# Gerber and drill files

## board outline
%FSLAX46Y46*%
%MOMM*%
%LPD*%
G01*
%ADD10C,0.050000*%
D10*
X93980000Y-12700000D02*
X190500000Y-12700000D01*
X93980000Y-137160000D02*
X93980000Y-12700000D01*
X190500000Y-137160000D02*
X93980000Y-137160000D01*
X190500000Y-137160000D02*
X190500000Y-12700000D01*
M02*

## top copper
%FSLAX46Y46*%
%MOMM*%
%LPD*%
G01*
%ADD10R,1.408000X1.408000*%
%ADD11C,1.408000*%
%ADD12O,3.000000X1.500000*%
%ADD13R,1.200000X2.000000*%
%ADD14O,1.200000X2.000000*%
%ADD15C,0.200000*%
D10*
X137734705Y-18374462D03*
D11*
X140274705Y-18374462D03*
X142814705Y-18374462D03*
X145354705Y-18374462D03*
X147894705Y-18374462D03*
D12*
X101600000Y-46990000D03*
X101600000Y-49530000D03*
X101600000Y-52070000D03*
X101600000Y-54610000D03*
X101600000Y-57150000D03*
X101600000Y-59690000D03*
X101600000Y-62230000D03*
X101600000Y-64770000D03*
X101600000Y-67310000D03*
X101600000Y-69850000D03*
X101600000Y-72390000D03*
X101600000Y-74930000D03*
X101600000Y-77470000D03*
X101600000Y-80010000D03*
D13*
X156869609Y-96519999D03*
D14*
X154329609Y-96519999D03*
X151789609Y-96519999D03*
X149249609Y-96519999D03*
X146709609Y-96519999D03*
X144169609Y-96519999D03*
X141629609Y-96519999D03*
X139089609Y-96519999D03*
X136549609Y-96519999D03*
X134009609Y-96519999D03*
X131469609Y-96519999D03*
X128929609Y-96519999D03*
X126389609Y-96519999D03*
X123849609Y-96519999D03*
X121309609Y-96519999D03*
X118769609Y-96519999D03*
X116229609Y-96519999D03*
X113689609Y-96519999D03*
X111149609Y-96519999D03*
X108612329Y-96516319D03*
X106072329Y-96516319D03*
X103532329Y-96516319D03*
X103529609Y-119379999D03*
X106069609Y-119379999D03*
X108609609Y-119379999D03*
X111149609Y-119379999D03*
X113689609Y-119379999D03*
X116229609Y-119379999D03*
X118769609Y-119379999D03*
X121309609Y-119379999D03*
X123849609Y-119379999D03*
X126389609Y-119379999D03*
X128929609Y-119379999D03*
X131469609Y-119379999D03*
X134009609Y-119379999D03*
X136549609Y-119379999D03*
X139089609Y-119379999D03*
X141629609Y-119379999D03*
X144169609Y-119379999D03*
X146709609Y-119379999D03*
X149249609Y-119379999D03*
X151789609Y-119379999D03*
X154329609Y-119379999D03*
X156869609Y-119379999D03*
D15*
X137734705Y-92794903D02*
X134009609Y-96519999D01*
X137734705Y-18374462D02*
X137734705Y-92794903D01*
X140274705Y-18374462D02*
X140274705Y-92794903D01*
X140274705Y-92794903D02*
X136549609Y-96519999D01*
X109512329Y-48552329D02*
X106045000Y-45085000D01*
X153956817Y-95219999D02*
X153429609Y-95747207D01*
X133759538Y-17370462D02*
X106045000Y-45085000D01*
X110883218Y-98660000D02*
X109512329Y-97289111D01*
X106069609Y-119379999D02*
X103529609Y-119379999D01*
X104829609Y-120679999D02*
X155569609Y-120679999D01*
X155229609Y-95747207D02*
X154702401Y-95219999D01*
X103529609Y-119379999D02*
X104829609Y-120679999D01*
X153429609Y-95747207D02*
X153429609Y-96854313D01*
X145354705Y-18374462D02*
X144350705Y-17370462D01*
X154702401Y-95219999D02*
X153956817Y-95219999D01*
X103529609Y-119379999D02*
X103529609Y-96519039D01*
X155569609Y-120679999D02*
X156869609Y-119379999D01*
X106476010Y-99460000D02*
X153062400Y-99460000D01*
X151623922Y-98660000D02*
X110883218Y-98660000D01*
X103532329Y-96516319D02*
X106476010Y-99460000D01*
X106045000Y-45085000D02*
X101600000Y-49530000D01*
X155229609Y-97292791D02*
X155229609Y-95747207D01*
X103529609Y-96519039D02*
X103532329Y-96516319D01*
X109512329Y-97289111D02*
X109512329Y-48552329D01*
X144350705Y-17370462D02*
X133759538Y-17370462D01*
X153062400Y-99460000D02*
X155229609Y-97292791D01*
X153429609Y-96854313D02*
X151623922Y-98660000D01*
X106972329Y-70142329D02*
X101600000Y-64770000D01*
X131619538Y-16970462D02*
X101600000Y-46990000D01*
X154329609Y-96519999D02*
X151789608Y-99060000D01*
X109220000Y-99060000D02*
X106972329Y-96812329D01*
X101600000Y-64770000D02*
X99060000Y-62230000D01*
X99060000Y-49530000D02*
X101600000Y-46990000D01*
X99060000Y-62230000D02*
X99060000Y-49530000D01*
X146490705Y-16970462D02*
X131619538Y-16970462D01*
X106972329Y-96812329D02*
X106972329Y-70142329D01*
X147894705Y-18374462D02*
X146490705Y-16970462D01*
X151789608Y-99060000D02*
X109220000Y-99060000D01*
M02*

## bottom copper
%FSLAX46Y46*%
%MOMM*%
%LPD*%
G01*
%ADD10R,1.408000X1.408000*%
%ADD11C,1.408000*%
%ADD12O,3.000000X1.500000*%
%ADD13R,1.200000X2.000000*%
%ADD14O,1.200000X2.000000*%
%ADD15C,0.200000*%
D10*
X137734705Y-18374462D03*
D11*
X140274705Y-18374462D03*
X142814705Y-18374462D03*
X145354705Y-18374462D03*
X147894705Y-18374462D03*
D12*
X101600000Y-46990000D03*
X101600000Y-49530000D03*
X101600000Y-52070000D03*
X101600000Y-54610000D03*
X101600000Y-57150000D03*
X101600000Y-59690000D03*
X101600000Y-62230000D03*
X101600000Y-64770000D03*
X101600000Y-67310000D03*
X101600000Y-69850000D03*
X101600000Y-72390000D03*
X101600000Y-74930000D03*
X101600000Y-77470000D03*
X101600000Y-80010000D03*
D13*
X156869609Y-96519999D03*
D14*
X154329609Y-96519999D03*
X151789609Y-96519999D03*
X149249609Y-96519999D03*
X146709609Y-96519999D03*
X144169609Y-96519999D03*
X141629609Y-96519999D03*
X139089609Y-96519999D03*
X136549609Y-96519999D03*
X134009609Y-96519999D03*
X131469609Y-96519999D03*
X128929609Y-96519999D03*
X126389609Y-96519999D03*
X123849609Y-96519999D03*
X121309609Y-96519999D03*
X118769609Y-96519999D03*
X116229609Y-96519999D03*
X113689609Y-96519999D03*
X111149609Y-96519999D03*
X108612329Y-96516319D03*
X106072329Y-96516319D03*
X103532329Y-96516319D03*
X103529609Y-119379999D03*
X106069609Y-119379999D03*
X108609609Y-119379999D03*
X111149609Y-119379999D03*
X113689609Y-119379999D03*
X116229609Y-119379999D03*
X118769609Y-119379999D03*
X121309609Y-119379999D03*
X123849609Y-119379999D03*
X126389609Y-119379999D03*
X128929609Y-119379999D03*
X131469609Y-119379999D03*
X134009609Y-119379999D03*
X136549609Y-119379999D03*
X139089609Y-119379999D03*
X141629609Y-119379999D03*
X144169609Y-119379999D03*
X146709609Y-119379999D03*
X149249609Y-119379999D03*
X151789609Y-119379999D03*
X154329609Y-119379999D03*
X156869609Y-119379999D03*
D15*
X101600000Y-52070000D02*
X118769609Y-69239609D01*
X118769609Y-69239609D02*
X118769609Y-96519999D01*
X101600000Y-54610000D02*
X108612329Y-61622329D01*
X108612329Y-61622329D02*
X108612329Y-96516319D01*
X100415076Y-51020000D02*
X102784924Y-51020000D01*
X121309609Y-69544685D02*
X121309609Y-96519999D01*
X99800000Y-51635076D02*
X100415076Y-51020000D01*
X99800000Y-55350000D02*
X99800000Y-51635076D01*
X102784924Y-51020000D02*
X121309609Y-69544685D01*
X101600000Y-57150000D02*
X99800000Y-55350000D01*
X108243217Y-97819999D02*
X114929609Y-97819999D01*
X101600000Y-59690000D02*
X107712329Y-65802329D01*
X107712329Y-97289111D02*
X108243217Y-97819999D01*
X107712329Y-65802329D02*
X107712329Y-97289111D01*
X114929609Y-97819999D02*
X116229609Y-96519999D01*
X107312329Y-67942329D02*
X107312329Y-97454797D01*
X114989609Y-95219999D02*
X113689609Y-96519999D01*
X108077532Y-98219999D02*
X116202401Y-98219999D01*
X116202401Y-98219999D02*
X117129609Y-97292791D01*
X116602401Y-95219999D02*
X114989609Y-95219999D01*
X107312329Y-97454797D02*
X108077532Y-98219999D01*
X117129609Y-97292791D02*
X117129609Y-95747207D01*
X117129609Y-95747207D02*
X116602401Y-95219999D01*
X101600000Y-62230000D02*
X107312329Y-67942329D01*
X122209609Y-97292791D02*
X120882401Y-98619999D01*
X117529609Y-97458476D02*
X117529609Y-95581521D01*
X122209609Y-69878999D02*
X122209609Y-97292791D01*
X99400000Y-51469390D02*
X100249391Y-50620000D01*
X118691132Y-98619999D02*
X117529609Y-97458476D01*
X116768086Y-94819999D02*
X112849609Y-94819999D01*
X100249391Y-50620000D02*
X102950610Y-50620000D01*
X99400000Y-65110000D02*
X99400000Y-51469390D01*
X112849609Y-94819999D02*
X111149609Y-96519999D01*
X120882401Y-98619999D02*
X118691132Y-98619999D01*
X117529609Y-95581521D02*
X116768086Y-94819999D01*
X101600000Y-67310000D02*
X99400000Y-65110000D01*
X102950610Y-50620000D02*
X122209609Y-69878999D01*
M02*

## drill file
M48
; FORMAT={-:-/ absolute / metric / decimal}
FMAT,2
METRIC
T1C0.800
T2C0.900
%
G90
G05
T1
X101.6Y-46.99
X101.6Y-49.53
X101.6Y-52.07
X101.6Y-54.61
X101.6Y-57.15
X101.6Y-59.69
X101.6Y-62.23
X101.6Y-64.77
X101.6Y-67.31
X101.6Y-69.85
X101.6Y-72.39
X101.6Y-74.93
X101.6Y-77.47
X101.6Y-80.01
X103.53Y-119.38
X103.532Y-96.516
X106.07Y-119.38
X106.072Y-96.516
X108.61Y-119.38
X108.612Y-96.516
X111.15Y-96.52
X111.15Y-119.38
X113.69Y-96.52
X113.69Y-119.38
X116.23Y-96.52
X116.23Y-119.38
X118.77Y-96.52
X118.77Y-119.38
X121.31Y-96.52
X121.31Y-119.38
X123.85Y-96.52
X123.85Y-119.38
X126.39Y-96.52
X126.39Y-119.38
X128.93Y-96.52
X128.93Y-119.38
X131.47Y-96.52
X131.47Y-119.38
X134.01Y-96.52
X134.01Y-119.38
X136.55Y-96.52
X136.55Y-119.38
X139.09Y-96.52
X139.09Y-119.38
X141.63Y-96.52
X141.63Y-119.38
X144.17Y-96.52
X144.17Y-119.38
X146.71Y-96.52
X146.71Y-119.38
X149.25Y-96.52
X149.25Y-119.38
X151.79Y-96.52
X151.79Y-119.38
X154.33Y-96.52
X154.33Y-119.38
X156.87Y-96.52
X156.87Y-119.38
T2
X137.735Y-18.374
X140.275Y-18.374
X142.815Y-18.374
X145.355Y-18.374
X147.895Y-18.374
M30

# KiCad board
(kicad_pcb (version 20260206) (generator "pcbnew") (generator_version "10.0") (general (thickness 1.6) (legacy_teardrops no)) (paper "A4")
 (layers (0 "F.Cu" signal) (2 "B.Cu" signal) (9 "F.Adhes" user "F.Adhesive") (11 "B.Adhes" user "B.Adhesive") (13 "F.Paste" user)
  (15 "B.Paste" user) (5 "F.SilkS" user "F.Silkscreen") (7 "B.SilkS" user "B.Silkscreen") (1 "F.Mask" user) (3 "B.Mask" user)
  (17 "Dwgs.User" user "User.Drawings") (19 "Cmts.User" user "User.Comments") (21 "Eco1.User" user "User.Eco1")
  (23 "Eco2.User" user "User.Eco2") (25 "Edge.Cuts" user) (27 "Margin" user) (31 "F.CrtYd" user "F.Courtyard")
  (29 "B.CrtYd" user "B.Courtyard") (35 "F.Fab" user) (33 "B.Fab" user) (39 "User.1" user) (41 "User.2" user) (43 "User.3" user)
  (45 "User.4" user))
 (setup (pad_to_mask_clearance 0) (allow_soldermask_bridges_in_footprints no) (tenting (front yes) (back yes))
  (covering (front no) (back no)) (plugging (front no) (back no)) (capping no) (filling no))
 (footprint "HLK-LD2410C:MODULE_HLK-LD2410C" (layer "F.Cu") (at 142.764705 24.914462)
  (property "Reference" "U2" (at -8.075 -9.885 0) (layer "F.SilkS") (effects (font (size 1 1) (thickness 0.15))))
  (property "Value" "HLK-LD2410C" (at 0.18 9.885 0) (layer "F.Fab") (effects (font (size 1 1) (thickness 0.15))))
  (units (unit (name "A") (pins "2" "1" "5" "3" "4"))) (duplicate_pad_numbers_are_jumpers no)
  (pad "1" thru_hole rect (at -5.03 -6.54) (size 1.408 1.408) (drill 0.9) (layers "*.Cu" "*.Mask") (remove_unused_layers no) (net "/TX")
   (solder_mask_margin 0.102))
  (pad "2" thru_hole circle (at -2.49 -6.54) (size 1.408 1.408) (drill 0.9) (layers "*.Cu" "*.Mask") (remove_unused_layers no) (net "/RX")
   (solder_mask_margin 0.102))
  (pad "3" thru_hole circle (at 0.05 -6.54) (size 1.408 1.408) (drill 0.9) (layers "*.Cu" "*.Mask") (remove_unused_layers no)
   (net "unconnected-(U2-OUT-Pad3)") (solder_mask_margin 0.102))
  (pad "4" thru_hole circle (at 2.59 -6.54) (size 1.408 1.408) (drill 0.9) (layers "*.Cu" "*.Mask") (remove_unused_layers no) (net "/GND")
   (solder_mask_margin 0.102))
  (pad "5" thru_hole circle (at 5.13 -6.54) (size 1.408 1.408) (drill 0.9) (layers "*.Cu" "*.Mask") (remove_unused_layers no) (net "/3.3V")
   (solder_mask_margin 0.102)))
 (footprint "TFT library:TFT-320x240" (layer "F.Cu") (at 101.6 63.5 -90)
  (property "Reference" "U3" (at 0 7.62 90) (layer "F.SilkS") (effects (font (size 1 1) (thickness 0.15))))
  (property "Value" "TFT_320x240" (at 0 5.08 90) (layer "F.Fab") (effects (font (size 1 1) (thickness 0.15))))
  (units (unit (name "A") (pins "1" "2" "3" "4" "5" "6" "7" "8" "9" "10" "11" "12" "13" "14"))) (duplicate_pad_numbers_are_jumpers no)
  (pad "1" thru_hole oval (at -16.51 0 270) (size 1.5 3) (drill 0.8) (layers "*.Cu" "*.Mask") (remove_unused_layers no) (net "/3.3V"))
  (pad "2" thru_hole oval (at -13.97 0 270) (size 1.5 3) (drill 0.8) (layers "*.Cu" "*.Mask") (remove_unused_layers no) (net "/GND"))
  (pad "3" thru_hole oval (at -11.43 0 270) (size 1.5 3) (drill 0.8) (layers "*.Cu" "*.Mask") (remove_unused_layers no) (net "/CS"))
  (pad "4" thru_hole oval (at -8.89 0 270) (size 1.5 3) (drill 0.8) (layers "*.Cu" "*.Mask") (remove_unused_layers no) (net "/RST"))
  (pad "5" thru_hole oval (at -6.35 0 270) (size 1.5 3) (drill 0.8) (layers "*.Cu" "*.Mask") (remove_unused_layers no) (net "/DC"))
  (pad "6" thru_hole oval (at -3.81 0 270) (size 1.5 3) (drill 0.8) (layers "*.Cu" "*.Mask") (remove_unused_layers no) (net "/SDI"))
  (pad "7" thru_hole oval (at -1.27 0 270) (size 1.5 3) (drill 0.8) (layers "*.Cu" "*.Mask") (remove_unused_layers no) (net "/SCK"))
  (pad "8" thru_hole oval (at 1.27 0 270) (size 1.5 3) (drill 0.8) (layers "*.Cu" "*.Mask") (remove_unused_layers no) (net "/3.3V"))
  (pad "9" thru_hole oval (at 3.81 0 270) (size 1.5 3) (drill 0.8) (layers "*.Cu" "*.Mask") (remove_unused_layers no) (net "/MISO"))
  (pad "10" thru_hole oval (at 6.35 0 270) (size 1.5 3) (drill 0.8) (layers "*.Cu" "*.Mask") (remove_unused_layers no)
   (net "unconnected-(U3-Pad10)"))
  (pad "11" thru_hole oval (at 8.89 0 270) (size 1.5 3) (drill 0.8) (layers "*.Cu" "*.Mask") (remove_unused_layers no)
   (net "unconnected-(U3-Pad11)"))
  (pad "12" thru_hole oval (at 11.43 0 270) (size 1.5 3) (drill 0.8) (layers "*.Cu" "*.Mask") (remove_unused_layers no)
   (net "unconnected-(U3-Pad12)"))
  (pad "13" thru_hole oval (at 13.97 0 270) (size 1.5 3) (drill 0.8) (layers "*.Cu" "*.Mask") (remove_unused_layers no)
   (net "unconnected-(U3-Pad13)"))
  (pad "14" thru_hole oval (at 16.51 0 270) (size 1.5 3) (drill 0.8) (layers "*.Cu" "*.Mask") (remove_unused_layers no)
   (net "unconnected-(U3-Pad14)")))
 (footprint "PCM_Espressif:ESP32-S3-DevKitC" (layer "F.Cu") (at 156.869609 96.519999 -90)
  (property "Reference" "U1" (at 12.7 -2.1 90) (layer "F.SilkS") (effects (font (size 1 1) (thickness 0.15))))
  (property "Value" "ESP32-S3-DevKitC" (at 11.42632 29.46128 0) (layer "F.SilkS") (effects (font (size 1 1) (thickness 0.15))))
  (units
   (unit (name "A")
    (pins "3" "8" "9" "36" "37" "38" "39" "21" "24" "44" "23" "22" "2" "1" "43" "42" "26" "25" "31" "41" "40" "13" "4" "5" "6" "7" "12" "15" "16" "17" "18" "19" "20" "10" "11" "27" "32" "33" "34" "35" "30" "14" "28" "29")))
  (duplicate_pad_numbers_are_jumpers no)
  (pad "1" thru_hole rect (at 0 0 180) (size 1.2 2) (drill 0.8) (layers "*.Cu" "*.Mask") (remove_unused_layers no) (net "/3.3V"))
  (pad "2" thru_hole oval (at 0 2.54 180) (size 1.2 2) (drill 0.8) (layers "*.Cu" "*.Mask") (remove_unused_layers no) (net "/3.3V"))
  (pad "3" thru_hole oval (at 0 5.08 180) (size 1.2 2) (drill 0.8) (layers "*.Cu" "*.Mask") (remove_unused_layers no)
   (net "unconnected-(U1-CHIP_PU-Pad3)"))
  (pad "4" thru_hole oval (at 0 7.62 180) (size 1.2 2) (drill 0.8) (layers "*.Cu" "*.Mask") (remove_unused_layers no)
   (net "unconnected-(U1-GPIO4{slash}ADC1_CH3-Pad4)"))
  (pad "5" thru_hole oval (at 0 10.16 180) (size 1.2 2) (drill 0.8) (layers "*.Cu" "*.Mask") (remove_unused_layers no)
   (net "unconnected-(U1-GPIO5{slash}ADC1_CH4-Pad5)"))
  (pad "6" thru_hole oval (at 0 12.7 180) (size 1.2 2) (drill 0.8) (layers "*.Cu" "*.Mask") (remove_unused_layers no)
   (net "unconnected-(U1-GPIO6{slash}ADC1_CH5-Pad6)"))
  (pad "7" thru_hole oval (at 0 15.24 180) (size 1.2 2) (drill 0.8) (layers "*.Cu" "*.Mask") (remove_unused_layers no)
   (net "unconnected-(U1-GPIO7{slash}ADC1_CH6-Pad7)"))
  (pad "8" thru_hole oval (at 0 17.78 180) (size 1.2 2) (drill 0.8) (layers "*.Cu" "*.Mask") (remove_unused_layers no)
   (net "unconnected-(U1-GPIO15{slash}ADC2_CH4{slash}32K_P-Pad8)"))
  (pad "9" thru_hole oval (at 0 20.32 180) (size 1.2 2) (drill 0.8) (layers "*.Cu" "*.Mask") (remove_unused_layers no) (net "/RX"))
  (pad "10" thru_hole oval (at 0 22.86 180) (size 1.2 2) (drill 0.8) (layers "*.Cu" "*.Mask") (remove_unused_layers no) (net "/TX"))
  (pad "11" thru_hole oval (at 0 25.4 180) (size 1.2 2) (drill 0.8) (layers "*.Cu" "*.Mask") (remove_unused_layers no)
   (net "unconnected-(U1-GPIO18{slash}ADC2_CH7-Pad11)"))
  (pad "12" thru_hole oval (at 0 27.94 180) (size 1.2 2) (drill 0.8) (layers "*.Cu" "*.Mask") (remove_unused_layers no)
   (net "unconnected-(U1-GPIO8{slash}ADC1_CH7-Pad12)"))
  (pad "13" thru_hole oval (at 0 30.48 180) (size 1.2 2) (drill 0.8) (layers "*.Cu" "*.Mask") (remove_unused_layers no)
   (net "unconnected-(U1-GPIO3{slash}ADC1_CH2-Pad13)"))
  (pad "14" thru_hole oval (at 0 33.02 180) (size 1.2 2) (drill 0.8) (layers "*.Cu" "*.Mask") (remove_unused_layers no)
   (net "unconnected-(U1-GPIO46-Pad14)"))
  (pad "15" thru_hole oval (at 0 35.56 180) (size 1.2 2) (drill 0.8) (layers "*.Cu" "*.Mask") (remove_unused_layers no) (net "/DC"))
  (pad "16" thru_hole oval (at 0 38.1 180) (size 1.2 2) (drill 0.8) (layers "*.Cu" "*.Mask") (remove_unused_layers no) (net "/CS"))
  (pad "17" thru_hole oval (at 0 40.64 180) (size 1.2 2) (drill 0.8) (layers "*.Cu" "*.Mask") (remove_unused_layers no) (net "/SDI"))
  (pad "18" thru_hole oval (at 0 43.18 180) (size 1.2 2) (drill 0.8) (layers "*.Cu" "*.Mask") (remove_unused_layers no) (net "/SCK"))
  (pad "19" thru_hole oval (at 0 45.72 180) (size 1.2 2) (drill 0.8) (layers "*.Cu" "*.Mask") (remove_unused_layers no) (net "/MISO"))
  (pad "20" thru_hole oval (at -0.00368 48.25728 180) (size 1.2 2) (drill 0.8) (layers "*.Cu" "*.Mask") (remove_unused_layers no)
   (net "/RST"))
  (pad "21" thru_hole oval (at -0.00368 50.79728 180) (size 1.2 2) (drill 0.8) (layers "*.Cu" "*.Mask") (remove_unused_layers no)
   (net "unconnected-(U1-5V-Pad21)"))
  (pad "22" thru_hole oval (at -0.00368 53.33728 180) (size 1.2 2) (drill 0.8) (layers "*.Cu" "*.Mask") (remove_unused_layers no)
   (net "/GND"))
  (pad "23" thru_hole oval (at 22.86 53.34 180) (size 1.2 2) (drill 0.8) (layers "*.Cu" "*.Mask") (remove_unused_layers no) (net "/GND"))
  (pad "24" thru_hole oval (at 22.86 50.8 180) (size 1.2 2) (drill 0.8) (layers "*.Cu" "*.Mask") (remove_unused_layers no) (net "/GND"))
  (pad "25" thru_hole oval (at 22.86 48.26 180) (size 1.2 2) (drill 0.8) (layers "*.Cu" "*.Mask") (remove_unused_layers no)
   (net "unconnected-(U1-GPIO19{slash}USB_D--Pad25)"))
  (pad "26" thru_hole oval (at 22.86 45.72 180) (size 1.2 2) (drill 0.8) (layers "*.Cu" "*.Mask") (remove_unused_layers no)
   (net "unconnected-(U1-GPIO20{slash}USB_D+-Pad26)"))
  (pad "27" thru_hole oval (at 22.86 43.18 180) (size 1.2 2) (drill 0.8) (layers "*.Cu" "*.Mask") (remove_unused_layers no)
   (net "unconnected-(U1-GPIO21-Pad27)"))
  (pad "28" thru_hole oval (at 22.86 40.64 180) (size 1.2 2) (drill 0.8) (layers "*.Cu" "*.Mask") (remove_unused_layers no)
   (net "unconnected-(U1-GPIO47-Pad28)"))
  (pad "29" thru_hole oval (at 22.86 38.1 180) (size 1.2 2) (drill 0.8) (layers "*.Cu" "*.Mask") (remove_unused_layers no)
   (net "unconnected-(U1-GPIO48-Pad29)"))
  (pad "30" thru_hole oval (at 22.86 35.56 180) (size 1.2 2) (drill 0.8) (layers "*.Cu" "*.Mask") (remove_unused_layers no)
   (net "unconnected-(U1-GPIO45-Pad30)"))
  (pad "31" thru_hole oval (at 22.86 33.02 180) (size 1.2 2) (drill 0.8) (layers "*.Cu" "*.Mask") (remove_unused_layers no)
   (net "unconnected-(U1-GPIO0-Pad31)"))
  (pad "32" thru_hole oval (at 22.86 30.48 180) (size 1.2 2) (drill 0.8) (layers "*.Cu" "*.Mask") (remove_unused_layers no)
   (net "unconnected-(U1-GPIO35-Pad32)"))
  (pad "33" thru_hole oval (at 22.86 27.94 180) (size 1.2 2) (drill 0.8) (layers "*.Cu" "*.Mask") (remove_unused_layers no)
   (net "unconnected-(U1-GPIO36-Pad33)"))
  (pad "34" thru_hole oval (at 22.86 25.4 180) (size 1.2 2) (drill 0.8) (layers "*.Cu" "*.Mask") (remove_unused_layers no)
   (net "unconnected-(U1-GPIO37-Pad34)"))
  (pad "35" thru_hole oval (at 22.86 22.86 180) (size 1.2 2) (drill 0.8) (layers "*.Cu" "*.Mask") (remove_unused_layers no)
   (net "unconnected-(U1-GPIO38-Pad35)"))
  (pad "36" thru_hole oval (at 22.86 20.32 180) (size 1.2 2) (drill 0.8) (layers "*.Cu" "*.Mask") (remove_unused_layers no)
   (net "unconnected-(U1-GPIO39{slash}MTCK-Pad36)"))
  (pad "37" thru_hole oval (at 22.86 17.78 180) (size 1.2 2) (drill 0.8) (layers "*.Cu" "*.Mask") (remove_unused_layers no)
   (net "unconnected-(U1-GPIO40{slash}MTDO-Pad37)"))
  (pad "38" thru_hole oval (at 22.86 15.24 180) (size 1.2 2) (drill 0.8) (layers "*.Cu" "*.Mask") (remove_unused_layers no)
   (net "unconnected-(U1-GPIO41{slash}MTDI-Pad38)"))
  (pad "39" thru_hole oval (at 22.86 12.7 180) (size 1.2 2) (drill 0.8) (layers "*.Cu" "*.Mask") (remove_unused_layers no)
   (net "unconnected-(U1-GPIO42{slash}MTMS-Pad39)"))
  (pad "40" thru_hole oval (at 22.86 10.16 180) (size 1.2 2) (drill 0.8) (layers "*.Cu" "*.Mask") (remove_unused_layers no)
   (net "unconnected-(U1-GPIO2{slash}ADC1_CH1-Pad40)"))
  (pad "41" thru_hole oval (at 22.86 7.62 180) (size 1.2 2) (drill 0.8) (layers "*.Cu" "*.Mask") (remove_unused_layers no)
   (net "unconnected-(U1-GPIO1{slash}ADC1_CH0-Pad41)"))
  (pad "42" thru_hole oval (at 22.86 5.08 180) (size 1.2 2) (drill 0.8) (layers "*.Cu" "*.Mask") (remove_unused_layers no)
   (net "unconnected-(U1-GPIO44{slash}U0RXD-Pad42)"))
  (pad "43" thru_hole oval (at 22.86 2.54 180) (size 1.2 2) (drill 0.8) (layers "*.Cu" "*.Mask") (remove_unused_layers no)
   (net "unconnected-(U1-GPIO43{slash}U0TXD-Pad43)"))
  (pad "44" thru_hole oval (at 22.86 0 180) (size 1.2 2) (drill 0.8) (layers "*.Cu" "*.Mask") (remove_unused_layers no) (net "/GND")))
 (gr_line (start 93.98 12.7) (end 190.5 12.7) (stroke (width 0.05) (type default)) (layer "Edge.Cuts"))
 (gr_line (start 93.98 137.16) (end 93.98 12.7) (stroke (width 0.05) (type default)) (layer "Edge.Cuts"))
 (gr_line (start 190.5 137.16) (end 93.98 137.16) (stroke (width 0.05) (type default)) (locked yes) (layer "Edge.Cuts"))
 (gr_line (start 190.5 137.16) (end 190.5 12.7) (stroke (width 0.05) (type default)) (layer "Edge.Cuts"))
 (segment (start 137.734705 92.794903) (end 134.009609 96.519999) (width 0.2) (layer "F.Cu") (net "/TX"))
 (segment (start 137.734705 18.374462) (end 137.734705 92.794903) (width 0.2) (layer "F.Cu") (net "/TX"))
 (segment (start 140.274705 18.374462) (end 140.274705 92.794903) (width 0.2) (layer "F.Cu") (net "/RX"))
 (segment (start 140.274705 92.794903) (end 136.549609 96.519999) (width 0.2) (layer "F.Cu") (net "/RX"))
 (segment (start 109.512329 48.552329) (end 106.045 45.085) (width 0.2) (layer "F.Cu") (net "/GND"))
 (segment (start 153.956817 95.219999) (end 153.429609 95.747207) (width 0.2) (layer "F.Cu") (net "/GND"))
 (segment (start 133.759538 17.370462) (end 106.045 45.085) (width 0.2) (layer "F.Cu") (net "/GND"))
 (segment (start 110.883218 98.66) (end 109.512329 97.289111) (width 0.2) (layer "F.Cu") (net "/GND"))
 (segment (start 106.069609 119.379999) (end 103.529609 119.379999) (width 0.2) (layer "F.Cu") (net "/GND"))
 (segment (start 104.829609 120.679999) (end 155.569609 120.679999) (width 0.2) (layer "F.Cu") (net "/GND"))
 (segment (start 155.229609 95.747207) (end 154.702401 95.219999) (width 0.2) (layer "F.Cu") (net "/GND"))
 (segment (start 103.529609 119.379999) (end 104.829609 120.679999) (width 0.2) (layer "F.Cu") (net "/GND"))
 (segment (start 153.429609 95.747207) (end 153.429609 96.854313) (width 0.2) (layer "F.Cu") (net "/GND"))
 (segment (start 145.354705 18.374462) (end 144.350705 17.370462) (width 0.2) (layer "F.Cu") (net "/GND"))
 (segment (start 154.702401 95.219999) (end 153.956817 95.219999) (width 0.2) (layer "F.Cu") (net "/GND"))
 (segment (start 103.529609 119.379999) (end 103.529609 96.519039) (width 0.2) (layer "F.Cu") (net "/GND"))
 (segment (start 155.569609 120.679999) (end 156.869609 119.379999) (width 0.2) (layer "F.Cu") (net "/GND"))
 (segment (start 106.47601 99.46) (end 153.0624 99.46) (width 0.2) (layer "F.Cu") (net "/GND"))
 (segment (start 151.623922 98.66) (end 110.883218 98.66) (width 0.2) (layer "F.Cu") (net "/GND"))
 (segment (start 103.532329 96.516319) (end 106.47601 99.46) (width 0.2) (layer "F.Cu") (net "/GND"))
 (segment (start 106.045 45.085) (end 101.6 49.53) (width 0.2) (layer "F.Cu") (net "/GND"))
 (segment (start 155.229609 97.292791) (end 155.229609 95.747207) (width 0.2) (layer "F.Cu") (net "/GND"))
 (segment (start 103.529609 96.519039) (end 103.532329 96.516319) (width 0.2) (layer "F.Cu") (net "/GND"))
 (segment (start 109.512329 97.289111) (end 109.512329 48.552329) (width 0.2) (layer "F.Cu") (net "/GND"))
 (segment (start 144.350705 17.370462) (end 133.759538 17.370462) (width 0.2) (layer "F.Cu") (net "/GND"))
 (segment (start 153.0624 99.46) (end 155.229609 97.292791) (width 0.2) (layer "F.Cu") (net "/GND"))
 (segment (start 153.429609 96.854313) (end 151.623922 98.66) (width 0.2) (layer "F.Cu") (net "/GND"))
 (segment (start 106.972329 70.142329) (end 101.6 64.77) (width 0.2) (layer "F.Cu") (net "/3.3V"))
 (segment (start 131.619538 16.970462) (end 101.6 46.99) (width 0.2) (layer "F.Cu") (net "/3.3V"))
 (segment (start 154.329609 96.519999) (end 151.789608 99.06) (width 0.2) (layer "F.Cu") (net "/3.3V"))
 (segment (start 109.22 99.06) (end 106.972329 96.812329) (width 0.2) (layer "F.Cu") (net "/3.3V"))
 (segment (start 101.6 64.77) (end 99.06 62.23) (width 0.2) (layer "F.Cu") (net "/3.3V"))
 (segment (start 99.06 49.53) (end 101.6 46.99) (width 0.2) (layer "F.Cu") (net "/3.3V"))
 (segment (start 99.06 62.23) (end 99.06 49.53) (width 0.2) (layer "F.Cu") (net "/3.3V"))
 (segment (start 146.490705 16.970462) (end 131.619538 16.970462) (width 0.2) (layer "F.Cu") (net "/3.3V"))
 (segment (start 106.972329 96.812329) (end 106.972329 70.142329) (width 0.2) (layer "F.Cu") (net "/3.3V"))
 (segment (start 147.894705 18.374462) (end 146.490705 16.970462) (width 0.2) (layer "F.Cu") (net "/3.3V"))
 (segment (start 151.789608 99.06) (end 109.22 99.06) (width 0.2) (layer "F.Cu") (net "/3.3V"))
 (segment (start 101.6 52.07) (end 118.769609 69.239609) (width 0.2) (layer "B.Cu") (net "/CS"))
 (segment (start 118.769609 69.239609) (end 118.769609 96.519999) (width 0.2) (layer "B.Cu") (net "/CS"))
 (segment (start 101.6 54.61) (end 108.612329 61.622329) (width 0.2) (layer "B.Cu") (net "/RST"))
 (segment (start 108.612329 61.622329) (end 108.612329 96.516319) (width 0.2) (layer "B.Cu") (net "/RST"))
 (segment (start 100.415076 51.02) (end 102.784924 51.02) (width 0.2) (layer "B.Cu") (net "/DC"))
 (segment (start 121.309609 69.544685) (end 121.309609 96.519999) (width 0.2) (layer "B.Cu") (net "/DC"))
 (segment (start 99.8 51.635076) (end 100.415076 51.02) (width 0.2) (layer "B.Cu") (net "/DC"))
 (segment (start 99.8 55.35) (end 99.8 51.635076) (width 0.2) (layer "B.Cu") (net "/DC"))
 (segment (start 102.784924 51.02) (end 121.309609 69.544685) (width 0.2) (layer "B.Cu") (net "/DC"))
 (segment (start 101.6 57.15) (end 99.8 55.35) (width 0.2) (layer "B.Cu") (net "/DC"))
 (segment (start 108.243217 97.819999) (end 114.929609 97.819999) (width 0.2) (layer "B.Cu") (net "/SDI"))
 (segment (start 101.6 59.69) (end 107.712329 65.802329) (width 0.2) (layer "B.Cu") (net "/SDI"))
 (segment (start 107.712329 97.289111) (end 108.243217 97.819999) (width 0.2) (layer "B.Cu") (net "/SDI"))
 (segment (start 107.712329 65.802329) (end 107.712329 97.289111) (width 0.2) (layer "B.Cu") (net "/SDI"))
 (segment (start 114.929609 97.819999) (end 116.229609 96.519999) (width 0.2) (layer "B.Cu") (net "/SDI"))
 (segment (start 107.312329 67.942329) (end 107.312329 97.454797) (width 0.2) (layer "B.Cu") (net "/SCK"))
 (segment (start 114.989609 95.219999) (end 113.689609 96.519999) (width 0.2) (layer "B.Cu") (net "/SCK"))
 (segment (start 108.077532 98.219999) (end 116.202401 98.219999) (width 0.2) (layer "B.Cu") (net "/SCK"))
 (segment (start 116.202401 98.219999) (end 117.129609 97.292791) (width 0.2) (layer "B.Cu") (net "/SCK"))
 (segment (start 116.602401 95.219999) (end 114.989609 95.219999) (width 0.2) (layer "B.Cu") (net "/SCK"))
 (segment (start 107.312329 97.454797) (end 108.077532 98.219999) (width 0.2) (layer "B.Cu") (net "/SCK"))
 (segment (start 117.129609 97.292791) (end 117.129609 95.747207) (width 0.2) (layer "B.Cu") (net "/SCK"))
 (segment (start 117.129609 95.747207) (end 116.602401 95.219999) (width 0.2) (layer "B.Cu") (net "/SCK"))
 (segment (start 101.6 62.23) (end 107.312329 67.942329) (width 0.2) (layer "B.Cu") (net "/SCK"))
 (segment (start 122.209609 97.292791) (end 120.882401 98.619999) (width 0.2) (layer "B.Cu") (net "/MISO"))
 (segment (start 117.529609 97.458476) (end 117.529609 95.581521) (width 0.2) (layer "B.Cu") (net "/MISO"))
 (segment (start 122.209609 69.878999) (end 122.209609 97.292791) (width 0.2) (layer "B.Cu") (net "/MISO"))
 (segment (start 99.4 51.46939) (end 100.249391 50.62) (width 0.2) (layer "B.Cu") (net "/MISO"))
 (segment (start 118.691132 98.619999) (end 117.529609 97.458476) (width 0.2) (layer "B.Cu") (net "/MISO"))
 (segment (start 116.768086 94.819999) (end 112.849609 94.819999) (width 0.2) (layer "B.Cu") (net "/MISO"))
 (segment (start 100.249391 50.62) (end 102.95061 50.62) (width 0.2) (layer "B.Cu") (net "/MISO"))
 (segment (start 99.4 65.11) (end 99.4 51.46939) (width 0.2) (layer "B.Cu") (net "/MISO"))
 (segment (start 112.849609 94.819999) (end 111.149609 96.519999) (width 0.2) (layer "B.Cu") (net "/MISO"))
 (segment (start 120.882401 98.619999) (end 118.691132 98.619999) (width 0.2) (layer "B.Cu") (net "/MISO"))
 (segment (start 117.529609 95.581521) (end 116.768086 94.819999) (width 0.2) (layer "B.Cu") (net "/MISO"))
 (segment (start 101.6 67.31) (end 99.4 65.11) (width 0.2) (layer "B.Cu") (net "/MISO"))
 (segment (start 102.95061 50.62) (end 122.209609 69.878999) (width 0.2) (layer "B.Cu") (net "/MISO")))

